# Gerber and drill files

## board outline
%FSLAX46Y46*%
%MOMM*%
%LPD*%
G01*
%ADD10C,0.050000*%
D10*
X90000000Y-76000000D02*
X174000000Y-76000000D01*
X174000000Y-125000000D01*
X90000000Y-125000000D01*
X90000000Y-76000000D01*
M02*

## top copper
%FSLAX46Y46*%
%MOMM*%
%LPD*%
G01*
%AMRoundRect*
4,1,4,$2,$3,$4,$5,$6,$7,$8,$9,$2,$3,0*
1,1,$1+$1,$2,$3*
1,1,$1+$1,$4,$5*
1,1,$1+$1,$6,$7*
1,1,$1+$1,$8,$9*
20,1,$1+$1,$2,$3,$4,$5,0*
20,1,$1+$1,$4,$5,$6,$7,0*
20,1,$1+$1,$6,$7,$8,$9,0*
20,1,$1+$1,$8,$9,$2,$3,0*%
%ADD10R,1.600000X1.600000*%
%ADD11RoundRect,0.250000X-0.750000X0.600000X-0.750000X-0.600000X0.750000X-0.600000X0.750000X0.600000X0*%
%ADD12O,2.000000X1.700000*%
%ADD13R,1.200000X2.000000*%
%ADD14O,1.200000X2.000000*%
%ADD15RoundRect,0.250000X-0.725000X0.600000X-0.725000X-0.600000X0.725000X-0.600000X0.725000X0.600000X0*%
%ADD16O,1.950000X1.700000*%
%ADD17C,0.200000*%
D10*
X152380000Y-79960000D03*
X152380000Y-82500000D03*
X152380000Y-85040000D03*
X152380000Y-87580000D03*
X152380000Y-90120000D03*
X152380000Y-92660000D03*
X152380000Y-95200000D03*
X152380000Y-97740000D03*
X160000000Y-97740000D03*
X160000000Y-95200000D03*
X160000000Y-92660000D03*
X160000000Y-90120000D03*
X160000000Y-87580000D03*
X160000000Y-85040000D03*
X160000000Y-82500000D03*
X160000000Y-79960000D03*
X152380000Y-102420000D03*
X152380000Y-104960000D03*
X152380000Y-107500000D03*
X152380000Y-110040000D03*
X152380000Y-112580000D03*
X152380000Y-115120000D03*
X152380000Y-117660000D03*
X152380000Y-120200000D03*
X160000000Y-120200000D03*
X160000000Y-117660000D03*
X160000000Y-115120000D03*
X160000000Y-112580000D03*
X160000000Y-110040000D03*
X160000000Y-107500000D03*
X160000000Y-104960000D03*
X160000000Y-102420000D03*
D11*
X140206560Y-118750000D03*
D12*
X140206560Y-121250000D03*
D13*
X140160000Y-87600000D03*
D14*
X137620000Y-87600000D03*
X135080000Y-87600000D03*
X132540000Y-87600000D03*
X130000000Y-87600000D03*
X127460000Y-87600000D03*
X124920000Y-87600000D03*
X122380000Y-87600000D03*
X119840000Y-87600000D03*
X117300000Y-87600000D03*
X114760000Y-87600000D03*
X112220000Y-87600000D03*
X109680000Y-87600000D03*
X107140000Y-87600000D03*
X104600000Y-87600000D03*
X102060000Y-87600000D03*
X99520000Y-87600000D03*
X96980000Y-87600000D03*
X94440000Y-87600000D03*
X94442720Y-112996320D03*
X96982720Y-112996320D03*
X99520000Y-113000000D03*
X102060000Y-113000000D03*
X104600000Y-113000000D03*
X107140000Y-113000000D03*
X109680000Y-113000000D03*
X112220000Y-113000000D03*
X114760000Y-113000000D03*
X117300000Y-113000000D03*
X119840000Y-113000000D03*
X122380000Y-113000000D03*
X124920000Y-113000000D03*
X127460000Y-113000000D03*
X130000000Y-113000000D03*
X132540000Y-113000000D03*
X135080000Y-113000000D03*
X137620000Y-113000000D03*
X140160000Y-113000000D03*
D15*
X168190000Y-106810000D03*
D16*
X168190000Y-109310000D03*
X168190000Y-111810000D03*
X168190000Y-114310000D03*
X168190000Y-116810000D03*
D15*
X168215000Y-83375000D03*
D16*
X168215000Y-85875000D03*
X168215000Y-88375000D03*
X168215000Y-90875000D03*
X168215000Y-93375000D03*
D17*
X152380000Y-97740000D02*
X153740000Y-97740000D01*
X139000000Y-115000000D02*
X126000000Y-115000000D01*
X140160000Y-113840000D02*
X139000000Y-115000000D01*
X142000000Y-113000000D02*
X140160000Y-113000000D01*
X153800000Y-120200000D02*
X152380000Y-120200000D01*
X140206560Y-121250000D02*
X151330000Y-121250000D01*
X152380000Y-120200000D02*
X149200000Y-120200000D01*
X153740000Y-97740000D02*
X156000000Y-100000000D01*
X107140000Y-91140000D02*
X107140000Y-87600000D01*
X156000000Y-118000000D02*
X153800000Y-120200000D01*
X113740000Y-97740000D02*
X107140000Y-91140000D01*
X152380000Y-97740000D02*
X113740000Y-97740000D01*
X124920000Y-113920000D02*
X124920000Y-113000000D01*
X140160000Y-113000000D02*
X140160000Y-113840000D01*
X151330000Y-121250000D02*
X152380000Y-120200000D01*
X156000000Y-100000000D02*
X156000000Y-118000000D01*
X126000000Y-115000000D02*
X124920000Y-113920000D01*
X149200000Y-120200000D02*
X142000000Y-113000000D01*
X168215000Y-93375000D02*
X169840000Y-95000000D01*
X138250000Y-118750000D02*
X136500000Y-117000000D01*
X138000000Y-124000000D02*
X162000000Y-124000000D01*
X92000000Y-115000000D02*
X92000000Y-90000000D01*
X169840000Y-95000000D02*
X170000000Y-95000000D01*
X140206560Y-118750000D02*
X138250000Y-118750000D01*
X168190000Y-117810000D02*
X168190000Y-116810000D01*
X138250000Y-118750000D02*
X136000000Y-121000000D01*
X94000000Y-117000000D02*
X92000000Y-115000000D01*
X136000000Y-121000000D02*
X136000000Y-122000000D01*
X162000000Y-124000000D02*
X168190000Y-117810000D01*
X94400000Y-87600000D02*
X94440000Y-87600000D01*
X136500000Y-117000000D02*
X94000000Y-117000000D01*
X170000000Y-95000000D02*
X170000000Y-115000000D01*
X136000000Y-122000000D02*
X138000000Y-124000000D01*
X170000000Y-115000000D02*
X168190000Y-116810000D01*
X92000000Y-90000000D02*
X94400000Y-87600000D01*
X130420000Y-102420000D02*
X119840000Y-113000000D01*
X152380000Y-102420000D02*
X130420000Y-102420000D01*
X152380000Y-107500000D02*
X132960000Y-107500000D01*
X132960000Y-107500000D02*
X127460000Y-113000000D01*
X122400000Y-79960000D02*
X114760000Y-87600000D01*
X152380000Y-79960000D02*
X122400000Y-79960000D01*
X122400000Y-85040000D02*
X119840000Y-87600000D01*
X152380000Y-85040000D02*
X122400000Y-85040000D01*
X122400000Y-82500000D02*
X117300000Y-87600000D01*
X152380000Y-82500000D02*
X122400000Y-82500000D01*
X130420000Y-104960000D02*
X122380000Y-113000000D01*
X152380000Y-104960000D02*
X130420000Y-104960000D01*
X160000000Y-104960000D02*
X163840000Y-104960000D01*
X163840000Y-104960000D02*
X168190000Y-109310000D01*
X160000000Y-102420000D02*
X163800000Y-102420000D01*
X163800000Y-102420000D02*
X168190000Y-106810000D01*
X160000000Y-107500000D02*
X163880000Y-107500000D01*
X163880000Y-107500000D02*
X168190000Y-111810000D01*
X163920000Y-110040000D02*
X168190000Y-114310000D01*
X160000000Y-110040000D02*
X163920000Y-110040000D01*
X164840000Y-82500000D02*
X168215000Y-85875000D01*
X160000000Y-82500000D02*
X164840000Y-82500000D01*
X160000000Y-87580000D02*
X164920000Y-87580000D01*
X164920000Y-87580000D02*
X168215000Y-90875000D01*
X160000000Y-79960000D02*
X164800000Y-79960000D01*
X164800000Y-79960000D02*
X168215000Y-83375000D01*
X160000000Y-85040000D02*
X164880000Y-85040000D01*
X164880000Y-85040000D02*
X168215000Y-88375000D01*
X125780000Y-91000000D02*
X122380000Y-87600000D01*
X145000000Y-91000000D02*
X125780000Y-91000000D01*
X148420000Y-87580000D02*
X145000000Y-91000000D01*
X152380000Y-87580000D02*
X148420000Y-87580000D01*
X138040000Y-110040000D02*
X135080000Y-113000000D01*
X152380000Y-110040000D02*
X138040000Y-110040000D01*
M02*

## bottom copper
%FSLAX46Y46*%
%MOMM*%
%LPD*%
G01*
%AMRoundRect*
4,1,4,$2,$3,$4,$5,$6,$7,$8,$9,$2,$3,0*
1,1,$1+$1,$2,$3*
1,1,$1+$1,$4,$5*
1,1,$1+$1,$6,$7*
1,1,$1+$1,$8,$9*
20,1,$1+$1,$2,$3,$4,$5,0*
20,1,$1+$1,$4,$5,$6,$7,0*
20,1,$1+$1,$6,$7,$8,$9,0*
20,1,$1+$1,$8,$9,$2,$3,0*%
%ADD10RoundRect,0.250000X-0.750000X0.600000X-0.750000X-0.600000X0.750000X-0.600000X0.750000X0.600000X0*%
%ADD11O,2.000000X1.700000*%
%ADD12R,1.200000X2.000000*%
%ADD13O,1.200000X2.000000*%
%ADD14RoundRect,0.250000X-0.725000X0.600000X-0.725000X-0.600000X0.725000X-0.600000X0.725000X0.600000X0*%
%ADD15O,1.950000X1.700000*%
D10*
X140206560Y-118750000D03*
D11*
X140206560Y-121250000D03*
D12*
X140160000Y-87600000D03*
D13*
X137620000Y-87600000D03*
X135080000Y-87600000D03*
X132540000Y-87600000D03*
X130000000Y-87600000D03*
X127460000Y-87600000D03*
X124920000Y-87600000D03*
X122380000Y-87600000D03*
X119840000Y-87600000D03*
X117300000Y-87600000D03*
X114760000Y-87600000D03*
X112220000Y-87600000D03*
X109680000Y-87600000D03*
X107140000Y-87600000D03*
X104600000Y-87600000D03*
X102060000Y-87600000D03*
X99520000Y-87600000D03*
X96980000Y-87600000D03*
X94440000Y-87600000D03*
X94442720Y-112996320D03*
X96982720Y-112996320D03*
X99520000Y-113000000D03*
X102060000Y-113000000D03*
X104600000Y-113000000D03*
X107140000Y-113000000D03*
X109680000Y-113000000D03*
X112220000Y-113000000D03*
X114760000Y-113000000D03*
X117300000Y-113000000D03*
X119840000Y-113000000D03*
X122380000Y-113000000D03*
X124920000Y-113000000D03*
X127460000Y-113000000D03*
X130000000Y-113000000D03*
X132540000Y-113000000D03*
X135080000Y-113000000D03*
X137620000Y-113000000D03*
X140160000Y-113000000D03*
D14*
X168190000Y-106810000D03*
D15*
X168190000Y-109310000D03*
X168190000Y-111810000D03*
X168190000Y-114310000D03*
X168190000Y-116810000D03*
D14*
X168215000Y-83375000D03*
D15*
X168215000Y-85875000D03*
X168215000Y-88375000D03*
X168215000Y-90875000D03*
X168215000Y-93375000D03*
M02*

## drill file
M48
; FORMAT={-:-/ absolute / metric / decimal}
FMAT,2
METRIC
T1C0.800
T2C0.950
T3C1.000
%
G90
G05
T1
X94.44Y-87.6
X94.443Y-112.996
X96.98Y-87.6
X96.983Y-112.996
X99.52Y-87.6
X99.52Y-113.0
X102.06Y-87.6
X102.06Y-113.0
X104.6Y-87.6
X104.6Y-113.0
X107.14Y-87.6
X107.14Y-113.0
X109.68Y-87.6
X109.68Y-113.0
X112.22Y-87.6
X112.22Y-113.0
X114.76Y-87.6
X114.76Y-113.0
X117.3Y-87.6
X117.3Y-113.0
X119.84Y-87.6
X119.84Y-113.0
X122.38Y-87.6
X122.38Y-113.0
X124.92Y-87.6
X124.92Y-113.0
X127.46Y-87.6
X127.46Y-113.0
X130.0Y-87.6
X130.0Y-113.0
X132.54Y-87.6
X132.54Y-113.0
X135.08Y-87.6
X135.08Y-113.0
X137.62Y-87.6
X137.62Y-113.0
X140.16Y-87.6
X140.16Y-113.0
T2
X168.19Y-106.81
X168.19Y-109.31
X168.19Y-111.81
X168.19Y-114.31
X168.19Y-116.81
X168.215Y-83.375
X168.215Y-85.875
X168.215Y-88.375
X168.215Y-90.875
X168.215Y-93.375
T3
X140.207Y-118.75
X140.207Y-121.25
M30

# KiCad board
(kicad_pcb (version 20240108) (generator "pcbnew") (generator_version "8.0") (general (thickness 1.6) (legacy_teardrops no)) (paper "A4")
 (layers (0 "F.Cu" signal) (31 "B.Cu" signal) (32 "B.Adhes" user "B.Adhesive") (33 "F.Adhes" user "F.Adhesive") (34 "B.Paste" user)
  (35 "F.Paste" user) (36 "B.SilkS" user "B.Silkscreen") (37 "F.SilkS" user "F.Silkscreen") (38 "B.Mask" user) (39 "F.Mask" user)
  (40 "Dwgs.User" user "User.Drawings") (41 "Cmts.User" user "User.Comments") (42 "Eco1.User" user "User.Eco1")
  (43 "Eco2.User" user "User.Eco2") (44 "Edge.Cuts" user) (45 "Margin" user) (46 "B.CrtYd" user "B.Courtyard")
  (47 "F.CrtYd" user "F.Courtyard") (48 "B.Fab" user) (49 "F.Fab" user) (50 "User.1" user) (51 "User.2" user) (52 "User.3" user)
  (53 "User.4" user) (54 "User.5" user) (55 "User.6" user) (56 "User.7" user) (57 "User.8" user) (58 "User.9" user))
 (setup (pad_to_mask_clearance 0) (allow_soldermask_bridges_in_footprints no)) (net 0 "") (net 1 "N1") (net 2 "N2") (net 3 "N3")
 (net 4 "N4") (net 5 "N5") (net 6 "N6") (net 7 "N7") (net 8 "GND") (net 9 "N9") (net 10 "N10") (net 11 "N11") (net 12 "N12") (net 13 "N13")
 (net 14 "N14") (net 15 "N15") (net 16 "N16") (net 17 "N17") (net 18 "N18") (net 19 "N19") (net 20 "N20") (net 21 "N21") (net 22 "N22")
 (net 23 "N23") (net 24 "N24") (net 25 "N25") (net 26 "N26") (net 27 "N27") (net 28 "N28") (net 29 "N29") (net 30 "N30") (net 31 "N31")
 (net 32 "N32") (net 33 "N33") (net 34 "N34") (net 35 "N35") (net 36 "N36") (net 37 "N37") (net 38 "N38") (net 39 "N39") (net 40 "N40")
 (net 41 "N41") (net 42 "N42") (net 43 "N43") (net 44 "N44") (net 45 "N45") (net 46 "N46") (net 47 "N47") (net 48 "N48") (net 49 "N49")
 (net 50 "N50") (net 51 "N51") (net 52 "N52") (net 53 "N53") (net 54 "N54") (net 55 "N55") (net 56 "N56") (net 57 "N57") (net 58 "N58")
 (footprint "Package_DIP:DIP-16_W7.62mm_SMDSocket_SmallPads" (layer "F.Cu") (at 156.19 88.85)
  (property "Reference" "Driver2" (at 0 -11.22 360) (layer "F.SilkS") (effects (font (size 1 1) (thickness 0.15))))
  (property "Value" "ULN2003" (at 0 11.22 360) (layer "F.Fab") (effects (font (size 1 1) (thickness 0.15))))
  (pad "1" smd rect (at -3.81 -8.89) (size 1.6 1.6) (layers "F.Cu" "F.Paste" "F.Mask") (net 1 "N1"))
  (pad "2" smd rect (at -3.81 -6.35) (size 1.6 1.6) (layers "F.Cu" "F.Paste" "F.Mask") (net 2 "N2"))
  (pad "3" smd rect (at -3.81 -3.81) (size 1.6 1.6) (layers "F.Cu" "F.Paste" "F.Mask") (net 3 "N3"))
  (pad "4" smd rect (at -3.81 -1.27) (size 1.6 1.6) (layers "F.Cu" "F.Paste" "F.Mask") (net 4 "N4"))
  (pad "5" smd rect (at -3.81 1.27) (size 1.6 1.6) (layers "F.Cu" "F.Paste" "F.Mask") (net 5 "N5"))
  (pad "6" smd rect (at -3.81 3.81) (size 1.6 1.6) (layers "F.Cu" "F.Paste" "F.Mask") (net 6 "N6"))
  (pad "7" smd rect (at -3.81 6.35) (size 1.6 1.6) (layers "F.Cu" "F.Paste" "F.Mask") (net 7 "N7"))
  (pad "8" smd rect (at -3.81 8.89) (size 1.6 1.6) (layers "F.Cu" "F.Paste" "F.Mask") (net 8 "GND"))
  (pad "9" smd rect (at 3.81 8.89) (size 1.6 1.6) (layers "F.Cu" "F.Paste" "F.Mask") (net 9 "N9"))
  (pad "10" smd rect (at 3.81 6.35) (size 1.6 1.6) (layers "F.Cu" "F.Paste" "F.Mask") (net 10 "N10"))
  (pad "11" smd rect (at 3.81 3.81) (size 1.6 1.6) (layers "F.Cu" "F.Paste" "F.Mask") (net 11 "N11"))
  (pad "12" smd rect (at 3.81 1.27) (size 1.6 1.6) (layers "F.Cu" "F.Paste" "F.Mask") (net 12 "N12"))
  (pad "13" smd rect (at 3.81 -1.27) (size 1.6 1.6) (layers "F.Cu" "F.Paste" "F.Mask") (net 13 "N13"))
  (pad "14" smd rect (at 3.81 -3.81) (size 1.6 1.6) (layers "F.Cu" "F.Paste" "F.Mask") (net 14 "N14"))
  (pad "15" smd rect (at 3.81 -6.35) (size 1.6 1.6) (layers "F.Cu" "F.Paste" "F.Mask") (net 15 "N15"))
  (pad "16" smd rect (at 3.81 -8.89) (size 1.6 1.6) (layers "F.Cu" "F.Paste" "F.Mask") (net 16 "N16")))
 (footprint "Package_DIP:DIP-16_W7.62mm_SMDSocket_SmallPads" (layer "F.Cu") (at 156.19 111.31)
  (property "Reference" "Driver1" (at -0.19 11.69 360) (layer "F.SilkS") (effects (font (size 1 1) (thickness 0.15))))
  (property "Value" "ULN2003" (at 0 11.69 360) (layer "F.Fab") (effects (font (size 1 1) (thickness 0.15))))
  (pad "1" smd rect (at -3.81 -8.89) (size 1.6 1.6) (layers "F.Cu" "F.Paste" "F.Mask") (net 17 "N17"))
  (pad "2" smd rect (at -3.81 -6.35) (size 1.6 1.6) (layers "F.Cu" "F.Paste" "F.Mask") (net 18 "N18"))
  (pad "3" smd rect (at -3.81 -3.81) (size 1.6 1.6) (layers "F.Cu" "F.Paste" "F.Mask") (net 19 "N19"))
  (pad "4" smd rect (at -3.81 -1.27) (size 1.6 1.6) (layers "F.Cu" "F.Paste" "F.Mask") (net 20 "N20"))
  (pad "5" smd rect (at -3.81 1.27) (size 1.6 1.6) (layers "F.Cu" "F.Paste" "F.Mask") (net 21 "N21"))
  (pad "6" smd rect (at -3.81 3.81) (size 1.6 1.6) (layers "F.Cu" "F.Paste" "F.Mask") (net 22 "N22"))
  (pad "7" smd rect (at -3.81 6.35) (size 1.6 1.6) (layers "F.Cu" "F.Paste" "F.Mask") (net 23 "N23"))
  (pad "8" smd rect (at -3.81 8.89) (size 1.6 1.6) (layers "F.Cu" "F.Paste" "F.Mask") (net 8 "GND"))
  (pad "9" smd rect (at 3.81 8.89) (size 1.6 1.6) (layers "F.Cu" "F.Paste" "F.Mask") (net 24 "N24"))
  (pad "10" smd rect (at 3.81 6.35) (size 1.6 1.6) (layers "F.Cu" "F.Paste" "F.Mask") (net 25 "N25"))
  (pad "11" smd rect (at 3.81 3.81) (size 1.6 1.6) (layers "F.Cu" "F.Paste" "F.Mask") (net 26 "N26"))
  (pad "12" smd rect (at 3.81 1.27) (size 1.6 1.6) (layers "F.Cu" "F.Paste" "F.Mask") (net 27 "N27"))
  (pad "13" smd rect (at 3.81 -1.27) (size 1.6 1.6) (layers "F.Cu" "F.Paste" "F.Mask") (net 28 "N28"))
  (pad "14" smd rect (at 3.81 -3.81) (size 1.6 1.6) (layers "F.Cu" "F.Paste" "F.Mask") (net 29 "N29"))
  (pad "15" smd rect (at 3.81 -6.35) (size 1.6 1.6) (layers "F.Cu" "F.Paste" "F.Mask") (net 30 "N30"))
  (pad "16" smd rect (at 3.81 -8.89) (size 1.6 1.6) (layers "F.Cu" "F.Paste" "F.Mask") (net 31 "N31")))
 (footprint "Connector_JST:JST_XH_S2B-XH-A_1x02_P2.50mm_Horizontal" (layer "F.Cu") (at 140.20656 118.75 -90)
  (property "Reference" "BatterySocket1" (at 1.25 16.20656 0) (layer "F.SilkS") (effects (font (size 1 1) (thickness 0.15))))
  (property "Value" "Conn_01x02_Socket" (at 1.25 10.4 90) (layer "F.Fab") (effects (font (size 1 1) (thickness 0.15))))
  (pad "1" thru_hole roundrect (at 0 0 270) (size 1.7 2) (drill 1) (layers "*.Cu" "*.Mask") (remove_unused_layers no)
   (roundrect_rratio 0.147059) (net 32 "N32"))
  (pad "2" thru_hole oval (at 2.5 0 270) (size 1.7 2) (drill 1) (layers "*.Cu" "*.Mask") (remove_unused_layers no) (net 8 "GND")))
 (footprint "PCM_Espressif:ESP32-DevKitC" (layer "F.Cu") (at 140.16 87.6 -90)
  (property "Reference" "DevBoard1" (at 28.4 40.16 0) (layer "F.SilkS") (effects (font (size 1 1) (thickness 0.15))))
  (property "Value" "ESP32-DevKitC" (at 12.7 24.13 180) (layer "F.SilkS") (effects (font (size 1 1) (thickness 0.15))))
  (pad "1" thru_hole rect (at 0 0 180) (size 1.2 2) (drill 0.8) (layers "*.Cu" "*.Mask") (remove_unused_layers no) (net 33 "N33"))
  (pad "2" thru_hole oval (at 0 2.54 180) (size 1.2 2) (drill 0.8) (layers "*.Cu" "*.Mask") (remove_unused_layers no) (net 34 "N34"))
  (pad "3" thru_hole oval (at 0 5.08 180) (size 1.2 2) (drill 0.8) (layers "*.Cu" "*.Mask") (remove_unused_layers no) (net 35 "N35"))
  (pad "4" thru_hole oval (at 0 7.62 180) (size 1.2 2) (drill 0.8) (layers "*.Cu" "*.Mask") (remove_unused_layers no) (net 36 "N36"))
  (pad "5" thru_hole oval (at 0 10.16 180) (size 1.2 2) (drill 0.8) (layers "*.Cu" "*.Mask") (remove_unused_layers no) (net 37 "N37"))
  (pad "6" thru_hole oval (at 0 12.7 180) (size 1.2 2) (drill 0.8) (layers "*.Cu" "*.Mask") (remove_unused_layers no) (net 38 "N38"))
  (pad "7" thru_hole oval (at 0 15.24 180) (size 1.2 2) (drill 0.8) (layers "*.Cu" "*.Mask") (remove_unused_layers no) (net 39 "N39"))
  (pad "8" thru_hole oval (at 0 17.78 180) (size 1.2 2) (drill 0.8) (layers "*.Cu" "*.Mask") (remove_unused_layers no) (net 4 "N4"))
  (pad "9" thru_hole oval (at 0 20.32 180) (size 1.2 2) (drill 0.8) (layers "*.Cu" "*.Mask") (remove_unused_layers no) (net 3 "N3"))
  (pad "10" thru_hole oval (at 0 22.86 180) (size 1.2 2) (drill 0.8) (layers "*.Cu" "*.Mask") (remove_unused_layers no) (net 2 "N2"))
  (pad "11" thru_hole oval (at 0 25.4 180) (size 1.2 2) (drill 0.8) (layers "*.Cu" "*.Mask") (remove_unused_layers no) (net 1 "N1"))
  (pad "12" thru_hole oval (at 0 27.94 180) (size 1.2 2) (drill 0.8) (layers "*.Cu" "*.Mask") (remove_unused_layers no) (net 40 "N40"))
  (pad "13" thru_hole oval (at 0 30.48 180) (size 1.2 2) (drill 0.8) (layers "*.Cu" "*.Mask") (remove_unused_layers no) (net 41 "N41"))
  (pad "14" thru_hole oval (at 0 33.02 180) (size 1.2 2) (drill 0.8) (layers "*.Cu" "*.Mask") (remove_unused_layers no) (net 8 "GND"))
  (pad "15" thru_hole oval (at 0 35.56 180) (size 1.2 2) (drill 0.8) (layers "*.Cu" "*.Mask") (remove_unused_layers no) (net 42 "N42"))
  (pad "16" thru_hole oval (at 0 38.1 180) (size 1.2 2) (drill 0.8) (layers "*.Cu" "*.Mask") (remove_unused_layers no) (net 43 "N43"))
  (pad "17" thru_hole oval (at 0 40.64 180) (size 1.2 2) (drill 0.8) (layers "*.Cu" "*.Mask") (remove_unused_layers no) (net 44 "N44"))
  (pad "18" thru_hole oval (at 0 43.18 180) (size 1.2 2) (drill 0.8) (layers "*.Cu" "*.Mask") (remove_unused_layers no) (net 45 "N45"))
  (pad "19" thru_hole oval (at 0 45.72 180) (size 1.2 2) (drill 0.8) (layers "*.Cu" "*.Mask") (remove_unused_layers no) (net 32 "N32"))
  (pad "20" thru_hole oval (at 25.39632 45.71728 180) (size 1.2 2) (drill 0.8) (layers "*.Cu" "*.Mask") (remove_unused_layers no)
   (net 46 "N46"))
  (pad "21" thru_hole oval (at 25.39632 43.17728 180) (size 1.2 2) (drill 0.8) (layers "*.Cu" "*.Mask") (remove_unused_layers no)
   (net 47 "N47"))
  (pad "22" thru_hole oval (at 25.4 40.64 180) (size 1.2 2) (drill 0.8) (layers "*.Cu" "*.Mask") (remove_unused_layers no) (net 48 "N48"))
  (pad "23" thru_hole oval (at 25.4 38.1 180) (size 1.2 2) (drill 0.8) (layers "*.Cu" "*.Mask") (remove_unused_layers no) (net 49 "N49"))
  (pad "24" thru_hole oval (at 25.4 35.56 180) (size 1.2 2) (drill 0.8) (layers "*.Cu" "*.Mask") (remove_unused_layers no) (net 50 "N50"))
  (pad "25" thru_hole oval (at 25.4 33.02 180) (size 1.2 2) (drill 0.8) (layers "*.Cu" "*.Mask") (remove_unused_layers no) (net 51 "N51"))
  (pad "26" thru_hole oval (at 25.4 30.48 180) (size 1.2 2) (drill 0.8) (layers "*.Cu" "*.Mask") (remove_unused_layers no) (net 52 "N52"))
  (pad "27" thru_hole oval (at 25.4 27.94 180) (size 1.2 2) (drill 0.8) (layers "*.Cu" "*.Mask") (remove_unused_layers no) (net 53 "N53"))
  (pad "28" thru_hole oval (at 25.4 25.4 180) (size 1.2 2) (drill 0.8) (layers "*.Cu" "*.Mask") (remove_unused_layers no) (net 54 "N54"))
  (pad "29" thru_hole oval (at 25.4 22.86 180) (size 1.2 2) (drill 0.8) (layers "*.Cu" "*.Mask") (remove_unused_layers no) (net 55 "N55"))
  (pad "30" thru_hole oval (at 25.4 20.32 180) (size 1.2 2) (drill 0.8) (layers "*.Cu" "*.Mask") (remove_unused_layers no) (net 17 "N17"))
  (pad "31" thru_hole oval (at 25.4 17.78 180) (size 1.2 2) (drill 0.8) (layers "*.Cu" "*.Mask") (remove_unused_layers no) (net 18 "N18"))
  (pad "32" thru_hole oval (at 25.4 15.24 180) (size 1.2 2) (drill 0.8) (layers "*.Cu" "*.Mask") (remove_unused_layers no) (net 8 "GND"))
  (pad "33" thru_hole oval (at 25.4 12.7 180) (size 1.2 2) (drill 0.8) (layers "*.Cu" "*.Mask") (remove_unused_layers no) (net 19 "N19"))
  (pad "34" thru_hole oval (at 25.4 10.16 180) (size 1.2 2) (drill 0.8) (layers "*.Cu" "*.Mask") (remove_unused_layers no) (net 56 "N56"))
  (pad "35" thru_hole oval (at 25.4 7.62 180) (size 1.2 2) (drill 0.8) (layers "*.Cu" "*.Mask") (remove_unused_layers no) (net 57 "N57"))
  (pad "36" thru_hole oval (at 25.4 5.08 180) (size 1.2 2) (drill 0.8) (layers "*.Cu" "*.Mask") (remove_unused_layers no) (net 20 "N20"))
  (pad "37" thru_hole oval (at 25.4 2.54 180) (size 1.2 2) (drill 0.8) (layers "*.Cu" "*.Mask") (remove_unused_layers no) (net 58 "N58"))
  (pad "38" thru_hole oval (at 25.4 0 180) (size 1.2 2) (drill 0.8) (layers "*.Cu" "*.Mask") (remove_unused_layers no) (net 8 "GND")))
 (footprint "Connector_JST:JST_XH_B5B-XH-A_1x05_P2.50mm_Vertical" (layer "F.Cu") (at 168.19 106.81 -90)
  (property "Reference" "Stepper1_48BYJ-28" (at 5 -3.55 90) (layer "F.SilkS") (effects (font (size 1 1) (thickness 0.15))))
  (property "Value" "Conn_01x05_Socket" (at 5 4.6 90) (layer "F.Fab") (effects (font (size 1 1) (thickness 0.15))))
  (pad "1" thru_hole roundrect (at 0 0 270) (size 1.7 1.95) (drill 0.95) (layers "*.Cu" "*.Mask") (remove_unused_layers no)
   (roundrect_rratio 0.147059) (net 31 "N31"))
  (pad "2" thru_hole oval (at 2.5 0 270) (size 1.7 1.95) (drill 0.95) (layers "*.Cu" "*.Mask") (remove_unused_layers no) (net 30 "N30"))
  (pad "3" thru_hole oval (at 5 0 270) (size 1.7 1.95) (drill 0.95) (layers "*.Cu" "*.Mask") (remove_unused_layers no) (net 29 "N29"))
  (pad "4" thru_hole oval (at 7.5 0 270) (size 1.7 1.95) (drill 0.95) (layers "*.Cu" "*.Mask") (remove_unused_layers no) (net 28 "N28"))
  (pad "5" thru_hole oval (at 10 0 270) (size 1.7 1.95) (drill 0.95) (layers "*.Cu" "*.Mask") (remove_unused_layers no) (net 32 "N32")))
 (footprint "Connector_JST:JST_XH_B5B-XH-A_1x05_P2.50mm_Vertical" (layer "F.Cu") (at 168.215 83.375 -90)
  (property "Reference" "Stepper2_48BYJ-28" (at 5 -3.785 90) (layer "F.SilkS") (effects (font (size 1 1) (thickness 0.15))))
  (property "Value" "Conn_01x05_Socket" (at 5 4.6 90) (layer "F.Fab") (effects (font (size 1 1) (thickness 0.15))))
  (pad "1" thru_hole roundrect (at 0 0 270) (size 1.7 1.95) (drill 0.95) (layers "*.Cu" "*.Mask") (remove_unused_layers no)
   (roundrect_rratio 0.147059) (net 16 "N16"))
  (pad "2" thru_hole oval (at 2.5 0 270) (size 1.7 1.95) (drill 0.95) (layers "*.Cu" "*.Mask") (remove_unused_layers no) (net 15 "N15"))
  (pad "3" thru_hole oval (at 5 0 270) (size 1.7 1.95) (drill 0.95) (layers "*.Cu" "*.Mask") (remove_unused_layers no) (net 14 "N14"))
  (pad "4" thru_hole oval (at 7.5 0 270) (size 1.7 1.95) (drill 0.95) (layers "*.Cu" "*.Mask") (remove_unused_layers no) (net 13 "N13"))
  (pad "5" thru_hole oval (at 10 0 270) (size 1.7 1.95) (drill 0.95) (layers "*.Cu" "*.Mask") (remove_unused_layers no) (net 32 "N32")))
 (gr_rect (start 90 76) (end 174 125) (stroke (width 0.05) (type default)) (fill none) (layer "Edge.Cuts"))
 (segment (start 152.38 97.74) (end 153.74 97.74) (width 0.2) (layer "F.Cu") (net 8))
 (segment (start 139 115) (end 126 115) (width 0.2) (layer "F.Cu") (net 8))
 (segment (start 140.16 113.84) (end 139 115) (width 0.2) (layer "F.Cu") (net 8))
 (segment (start 142 113) (end 140.16 113) (width 0.2) (layer "F.Cu") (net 8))
 (segment (start 153.8 120.2) (end 152.38 120.2) (width 0.2) (layer "F.Cu") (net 8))
 (segment (start 140.20656 121.25) (end 151.33 121.25) (width 0.2) (layer "F.Cu") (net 8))
 (segment (start 152.38 120.2) (end 149.2 120.2) (width 0.2) (layer "F.Cu") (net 8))
 (segment (start 153.74 97.74) (end 156 100) (width 0.2) (layer "F.Cu") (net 8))
 (segment (start 107.14 91.14) (end 107.14 87.6) (width 0.2) (layer "F.Cu") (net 8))
 (segment (start 156 118) (end 153.8 120.2) (width 0.2) (layer "F.Cu") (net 8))
 (segment (start 113.74 97.74) (end 107.14 91.14) (width 0.2) (layer "F.Cu") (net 8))
 (segment (start 152.38 97.74) (end 113.74 97.74) (width 0.2) (layer "F.Cu") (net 8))
 (segment (start 124.92 113.92) (end 124.92 113) (width 0.2) (layer "F.Cu") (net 8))
 (segment (start 140.16 113) (end 140.16 113.84) (width 0.2) (layer "F.Cu") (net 8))
 (segment (start 151.33 121.25) (end 152.38 120.2) (width 0.2) (layer "F.Cu") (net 8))
 (segment (start 156 100) (end 156 118) (width 0.2) (layer "F.Cu") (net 8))
 (segment (start 126 115) (end 124.92 113.92) (width 0.2) (layer "F.Cu") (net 8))
 (segment (start 149.2 120.2) (end 142 113) (width 0.2) (layer "F.Cu") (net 8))
 (segment (start 168.215 93.375) (end 169.84 95) (width 0.2) (layer "F.Cu") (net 32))
 (segment (start 138.25 118.75) (end 136.5 117) (width 0.2) (layer "F.Cu") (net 32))
 (segment (start 138 124) (end 162 124) (width 0.2) (layer "F.Cu") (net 32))
 (segment (start 92 115) (end 92 90) (width 0.2) (layer "F.Cu") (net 32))
 (segment (start 169.84 95) (end 170 95) (width 0.2) (layer "F.Cu") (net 32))
 (segment (start 140.20656 118.75) (end 138.25 118.75) (width 0.2) (layer "F.Cu") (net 32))
 (segment (start 168.19 117.81) (end 168.19 116.81) (width 0.2) (layer "F.Cu") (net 32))
 (segment (start 138.25 118.75) (end 136 121) (width 0.2) (layer "F.Cu") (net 32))
 (segment (start 94 117) (end 92 115) (width 0.2) (layer "F.Cu") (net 32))
 (segment (start 136 121) (end 136 122) (width 0.2) (layer "F.Cu") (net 32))
 (segment (start 162 124) (end 168.19 117.81) (width 0.2) (layer "F.Cu") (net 32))
 (segment (start 94.4 87.6) (end 94.44 87.6) (width 0.2) (layer "F.Cu") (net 32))
 (segment (start 136.5 117) (end 94 117) (width 0.2) (layer "F.Cu") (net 32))
 (segment (start 170 95) (end 170 115) (width 0.2) (layer "F.Cu") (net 32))
 (segment (start 136 122) (end 138 124) (width 0.2) (layer "F.Cu") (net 32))
 (segment (start 170 115) (end 168.19 116.81) (width 0.2) (layer "F.Cu") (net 32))
 (segment (start 92 90) (end 94.4 87.6) (width 0.2) (layer "F.Cu") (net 32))
 (segment (start 130.42 102.42) (end 119.84 113) (width 0.2) (layer "F.Cu") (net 17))
 (segment (start 152.38 102.42) (end 130.42 102.42) (width 0.2) (layer "F.Cu") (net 17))
 (segment (start 152.38 107.5) (end 132.96 107.5) (width 0.2) (layer "F.Cu") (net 19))
 (segment (start 132.96 107.5) (end 127.46 113) (width 0.2) (layer "F.Cu") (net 19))
 (segment (start 122.4 79.96) (end 114.76 87.6) (width 0.2) (layer "F.Cu") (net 1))
 (segment (start 152.38 79.96) (end 122.4 79.96) (width 0.2) (layer "F.Cu") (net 1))
 (segment (start 122.4 85.04) (end 119.84 87.6) (width 0.2) (layer "F.Cu") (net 3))
 (segment (start 152.38 85.04) (end 122.4 85.04) (width 0.2) (layer "F.Cu") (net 3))
 (segment (start 122.4 82.5) (end 117.3 87.6) (width 0.2) (layer "F.Cu") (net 2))
 (segment (start 152.38 82.5) (end 122.4 82.5) (width 0.2) (layer "F.Cu") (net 2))
 (segment (start 130.42 104.96) (end 122.38 113) (width 0.2) (layer "F.Cu") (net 18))
 (segment (start 152.38 104.96) (end 130.42 104.96) (width 0.2) (layer "F.Cu") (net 18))
 (segment (start 160 104.96) (end 163.84 104.96) (width 0.2) (layer "F.Cu") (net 30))
 (segment (start 163.84 104.96) (end 168.19 109.31) (width 0.2) (layer "F.Cu") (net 30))
 (segment (start 160 102.42) (end 163.8 102.42) (width 0.2) (layer "F.Cu") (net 31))
 (segment (start 163.8 102.42) (end 168.19 106.81) (width 0.2) (layer "F.Cu") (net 31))
 (segment (start 160 107.5) (end 163.88 107.5) (width 0.2) (layer "F.Cu") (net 29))
 (segment (start 163.88 107.5) (end 168.19 111.81) (width 0.2) (layer "F.Cu") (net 29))
 (segment (start 163.92 110.04) (end 168.19 114.31) (width 0.2) (layer "F.Cu") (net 28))
 (segment (start 160 110.04) (end 163.92 110.04) (width 0.2) (layer "F.Cu") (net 28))
 (segment (start 164.84 82.5) (end 168.215 85.875) (width 0.2) (layer "F.Cu") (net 15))
 (segment (start 160 82.5) (end 164.84 82.5) (width 0.2) (layer "F.Cu") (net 15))
 (segment (start 160 87.58) (end 164.92 87.58) (width 0.2) (layer "F.Cu") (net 13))
 (segment (start 164.92 87.58) (end 168.215 90.875) (width 0.2) (layer "F.Cu") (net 13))
 (segment (start 160 79.96) (end 164.8 79.96) (width 0.2) (layer "F.Cu") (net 16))
 (segment (start 164.8 79.96) (end 168.215 83.375) (width 0.2) (layer "F.Cu") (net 16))
 (segment (start 160 85.04) (end 164.88 85.04) (width 0.2) (layer "F.Cu") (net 14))
 (segment (start 164.88 85.04) (end 168.215 88.375) (width 0.2) (layer "F.Cu") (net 14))
 (segment (start 125.78 91) (end 122.38 87.6) (width 0.2) (layer "F.Cu") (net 4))
 (segment (start 145 91) (end 125.78 91) (width 0.2) (layer "F.Cu") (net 4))
 (segment (start 148.42 87.58) (end 145 91) (width 0.2) (layer "F.Cu") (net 4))
 (segment (start 152.38 87.58) (end 148.42 87.58) (width 0.2) (layer "F.Cu") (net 4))
 (segment (start 138.04 110.04) (end 135.08 113) (width 0.2) (layer "F.Cu") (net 20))
 (segment (start 152.38 110.04) (end 138.04 110.04) (width 0.2) (layer "F.Cu") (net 20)))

